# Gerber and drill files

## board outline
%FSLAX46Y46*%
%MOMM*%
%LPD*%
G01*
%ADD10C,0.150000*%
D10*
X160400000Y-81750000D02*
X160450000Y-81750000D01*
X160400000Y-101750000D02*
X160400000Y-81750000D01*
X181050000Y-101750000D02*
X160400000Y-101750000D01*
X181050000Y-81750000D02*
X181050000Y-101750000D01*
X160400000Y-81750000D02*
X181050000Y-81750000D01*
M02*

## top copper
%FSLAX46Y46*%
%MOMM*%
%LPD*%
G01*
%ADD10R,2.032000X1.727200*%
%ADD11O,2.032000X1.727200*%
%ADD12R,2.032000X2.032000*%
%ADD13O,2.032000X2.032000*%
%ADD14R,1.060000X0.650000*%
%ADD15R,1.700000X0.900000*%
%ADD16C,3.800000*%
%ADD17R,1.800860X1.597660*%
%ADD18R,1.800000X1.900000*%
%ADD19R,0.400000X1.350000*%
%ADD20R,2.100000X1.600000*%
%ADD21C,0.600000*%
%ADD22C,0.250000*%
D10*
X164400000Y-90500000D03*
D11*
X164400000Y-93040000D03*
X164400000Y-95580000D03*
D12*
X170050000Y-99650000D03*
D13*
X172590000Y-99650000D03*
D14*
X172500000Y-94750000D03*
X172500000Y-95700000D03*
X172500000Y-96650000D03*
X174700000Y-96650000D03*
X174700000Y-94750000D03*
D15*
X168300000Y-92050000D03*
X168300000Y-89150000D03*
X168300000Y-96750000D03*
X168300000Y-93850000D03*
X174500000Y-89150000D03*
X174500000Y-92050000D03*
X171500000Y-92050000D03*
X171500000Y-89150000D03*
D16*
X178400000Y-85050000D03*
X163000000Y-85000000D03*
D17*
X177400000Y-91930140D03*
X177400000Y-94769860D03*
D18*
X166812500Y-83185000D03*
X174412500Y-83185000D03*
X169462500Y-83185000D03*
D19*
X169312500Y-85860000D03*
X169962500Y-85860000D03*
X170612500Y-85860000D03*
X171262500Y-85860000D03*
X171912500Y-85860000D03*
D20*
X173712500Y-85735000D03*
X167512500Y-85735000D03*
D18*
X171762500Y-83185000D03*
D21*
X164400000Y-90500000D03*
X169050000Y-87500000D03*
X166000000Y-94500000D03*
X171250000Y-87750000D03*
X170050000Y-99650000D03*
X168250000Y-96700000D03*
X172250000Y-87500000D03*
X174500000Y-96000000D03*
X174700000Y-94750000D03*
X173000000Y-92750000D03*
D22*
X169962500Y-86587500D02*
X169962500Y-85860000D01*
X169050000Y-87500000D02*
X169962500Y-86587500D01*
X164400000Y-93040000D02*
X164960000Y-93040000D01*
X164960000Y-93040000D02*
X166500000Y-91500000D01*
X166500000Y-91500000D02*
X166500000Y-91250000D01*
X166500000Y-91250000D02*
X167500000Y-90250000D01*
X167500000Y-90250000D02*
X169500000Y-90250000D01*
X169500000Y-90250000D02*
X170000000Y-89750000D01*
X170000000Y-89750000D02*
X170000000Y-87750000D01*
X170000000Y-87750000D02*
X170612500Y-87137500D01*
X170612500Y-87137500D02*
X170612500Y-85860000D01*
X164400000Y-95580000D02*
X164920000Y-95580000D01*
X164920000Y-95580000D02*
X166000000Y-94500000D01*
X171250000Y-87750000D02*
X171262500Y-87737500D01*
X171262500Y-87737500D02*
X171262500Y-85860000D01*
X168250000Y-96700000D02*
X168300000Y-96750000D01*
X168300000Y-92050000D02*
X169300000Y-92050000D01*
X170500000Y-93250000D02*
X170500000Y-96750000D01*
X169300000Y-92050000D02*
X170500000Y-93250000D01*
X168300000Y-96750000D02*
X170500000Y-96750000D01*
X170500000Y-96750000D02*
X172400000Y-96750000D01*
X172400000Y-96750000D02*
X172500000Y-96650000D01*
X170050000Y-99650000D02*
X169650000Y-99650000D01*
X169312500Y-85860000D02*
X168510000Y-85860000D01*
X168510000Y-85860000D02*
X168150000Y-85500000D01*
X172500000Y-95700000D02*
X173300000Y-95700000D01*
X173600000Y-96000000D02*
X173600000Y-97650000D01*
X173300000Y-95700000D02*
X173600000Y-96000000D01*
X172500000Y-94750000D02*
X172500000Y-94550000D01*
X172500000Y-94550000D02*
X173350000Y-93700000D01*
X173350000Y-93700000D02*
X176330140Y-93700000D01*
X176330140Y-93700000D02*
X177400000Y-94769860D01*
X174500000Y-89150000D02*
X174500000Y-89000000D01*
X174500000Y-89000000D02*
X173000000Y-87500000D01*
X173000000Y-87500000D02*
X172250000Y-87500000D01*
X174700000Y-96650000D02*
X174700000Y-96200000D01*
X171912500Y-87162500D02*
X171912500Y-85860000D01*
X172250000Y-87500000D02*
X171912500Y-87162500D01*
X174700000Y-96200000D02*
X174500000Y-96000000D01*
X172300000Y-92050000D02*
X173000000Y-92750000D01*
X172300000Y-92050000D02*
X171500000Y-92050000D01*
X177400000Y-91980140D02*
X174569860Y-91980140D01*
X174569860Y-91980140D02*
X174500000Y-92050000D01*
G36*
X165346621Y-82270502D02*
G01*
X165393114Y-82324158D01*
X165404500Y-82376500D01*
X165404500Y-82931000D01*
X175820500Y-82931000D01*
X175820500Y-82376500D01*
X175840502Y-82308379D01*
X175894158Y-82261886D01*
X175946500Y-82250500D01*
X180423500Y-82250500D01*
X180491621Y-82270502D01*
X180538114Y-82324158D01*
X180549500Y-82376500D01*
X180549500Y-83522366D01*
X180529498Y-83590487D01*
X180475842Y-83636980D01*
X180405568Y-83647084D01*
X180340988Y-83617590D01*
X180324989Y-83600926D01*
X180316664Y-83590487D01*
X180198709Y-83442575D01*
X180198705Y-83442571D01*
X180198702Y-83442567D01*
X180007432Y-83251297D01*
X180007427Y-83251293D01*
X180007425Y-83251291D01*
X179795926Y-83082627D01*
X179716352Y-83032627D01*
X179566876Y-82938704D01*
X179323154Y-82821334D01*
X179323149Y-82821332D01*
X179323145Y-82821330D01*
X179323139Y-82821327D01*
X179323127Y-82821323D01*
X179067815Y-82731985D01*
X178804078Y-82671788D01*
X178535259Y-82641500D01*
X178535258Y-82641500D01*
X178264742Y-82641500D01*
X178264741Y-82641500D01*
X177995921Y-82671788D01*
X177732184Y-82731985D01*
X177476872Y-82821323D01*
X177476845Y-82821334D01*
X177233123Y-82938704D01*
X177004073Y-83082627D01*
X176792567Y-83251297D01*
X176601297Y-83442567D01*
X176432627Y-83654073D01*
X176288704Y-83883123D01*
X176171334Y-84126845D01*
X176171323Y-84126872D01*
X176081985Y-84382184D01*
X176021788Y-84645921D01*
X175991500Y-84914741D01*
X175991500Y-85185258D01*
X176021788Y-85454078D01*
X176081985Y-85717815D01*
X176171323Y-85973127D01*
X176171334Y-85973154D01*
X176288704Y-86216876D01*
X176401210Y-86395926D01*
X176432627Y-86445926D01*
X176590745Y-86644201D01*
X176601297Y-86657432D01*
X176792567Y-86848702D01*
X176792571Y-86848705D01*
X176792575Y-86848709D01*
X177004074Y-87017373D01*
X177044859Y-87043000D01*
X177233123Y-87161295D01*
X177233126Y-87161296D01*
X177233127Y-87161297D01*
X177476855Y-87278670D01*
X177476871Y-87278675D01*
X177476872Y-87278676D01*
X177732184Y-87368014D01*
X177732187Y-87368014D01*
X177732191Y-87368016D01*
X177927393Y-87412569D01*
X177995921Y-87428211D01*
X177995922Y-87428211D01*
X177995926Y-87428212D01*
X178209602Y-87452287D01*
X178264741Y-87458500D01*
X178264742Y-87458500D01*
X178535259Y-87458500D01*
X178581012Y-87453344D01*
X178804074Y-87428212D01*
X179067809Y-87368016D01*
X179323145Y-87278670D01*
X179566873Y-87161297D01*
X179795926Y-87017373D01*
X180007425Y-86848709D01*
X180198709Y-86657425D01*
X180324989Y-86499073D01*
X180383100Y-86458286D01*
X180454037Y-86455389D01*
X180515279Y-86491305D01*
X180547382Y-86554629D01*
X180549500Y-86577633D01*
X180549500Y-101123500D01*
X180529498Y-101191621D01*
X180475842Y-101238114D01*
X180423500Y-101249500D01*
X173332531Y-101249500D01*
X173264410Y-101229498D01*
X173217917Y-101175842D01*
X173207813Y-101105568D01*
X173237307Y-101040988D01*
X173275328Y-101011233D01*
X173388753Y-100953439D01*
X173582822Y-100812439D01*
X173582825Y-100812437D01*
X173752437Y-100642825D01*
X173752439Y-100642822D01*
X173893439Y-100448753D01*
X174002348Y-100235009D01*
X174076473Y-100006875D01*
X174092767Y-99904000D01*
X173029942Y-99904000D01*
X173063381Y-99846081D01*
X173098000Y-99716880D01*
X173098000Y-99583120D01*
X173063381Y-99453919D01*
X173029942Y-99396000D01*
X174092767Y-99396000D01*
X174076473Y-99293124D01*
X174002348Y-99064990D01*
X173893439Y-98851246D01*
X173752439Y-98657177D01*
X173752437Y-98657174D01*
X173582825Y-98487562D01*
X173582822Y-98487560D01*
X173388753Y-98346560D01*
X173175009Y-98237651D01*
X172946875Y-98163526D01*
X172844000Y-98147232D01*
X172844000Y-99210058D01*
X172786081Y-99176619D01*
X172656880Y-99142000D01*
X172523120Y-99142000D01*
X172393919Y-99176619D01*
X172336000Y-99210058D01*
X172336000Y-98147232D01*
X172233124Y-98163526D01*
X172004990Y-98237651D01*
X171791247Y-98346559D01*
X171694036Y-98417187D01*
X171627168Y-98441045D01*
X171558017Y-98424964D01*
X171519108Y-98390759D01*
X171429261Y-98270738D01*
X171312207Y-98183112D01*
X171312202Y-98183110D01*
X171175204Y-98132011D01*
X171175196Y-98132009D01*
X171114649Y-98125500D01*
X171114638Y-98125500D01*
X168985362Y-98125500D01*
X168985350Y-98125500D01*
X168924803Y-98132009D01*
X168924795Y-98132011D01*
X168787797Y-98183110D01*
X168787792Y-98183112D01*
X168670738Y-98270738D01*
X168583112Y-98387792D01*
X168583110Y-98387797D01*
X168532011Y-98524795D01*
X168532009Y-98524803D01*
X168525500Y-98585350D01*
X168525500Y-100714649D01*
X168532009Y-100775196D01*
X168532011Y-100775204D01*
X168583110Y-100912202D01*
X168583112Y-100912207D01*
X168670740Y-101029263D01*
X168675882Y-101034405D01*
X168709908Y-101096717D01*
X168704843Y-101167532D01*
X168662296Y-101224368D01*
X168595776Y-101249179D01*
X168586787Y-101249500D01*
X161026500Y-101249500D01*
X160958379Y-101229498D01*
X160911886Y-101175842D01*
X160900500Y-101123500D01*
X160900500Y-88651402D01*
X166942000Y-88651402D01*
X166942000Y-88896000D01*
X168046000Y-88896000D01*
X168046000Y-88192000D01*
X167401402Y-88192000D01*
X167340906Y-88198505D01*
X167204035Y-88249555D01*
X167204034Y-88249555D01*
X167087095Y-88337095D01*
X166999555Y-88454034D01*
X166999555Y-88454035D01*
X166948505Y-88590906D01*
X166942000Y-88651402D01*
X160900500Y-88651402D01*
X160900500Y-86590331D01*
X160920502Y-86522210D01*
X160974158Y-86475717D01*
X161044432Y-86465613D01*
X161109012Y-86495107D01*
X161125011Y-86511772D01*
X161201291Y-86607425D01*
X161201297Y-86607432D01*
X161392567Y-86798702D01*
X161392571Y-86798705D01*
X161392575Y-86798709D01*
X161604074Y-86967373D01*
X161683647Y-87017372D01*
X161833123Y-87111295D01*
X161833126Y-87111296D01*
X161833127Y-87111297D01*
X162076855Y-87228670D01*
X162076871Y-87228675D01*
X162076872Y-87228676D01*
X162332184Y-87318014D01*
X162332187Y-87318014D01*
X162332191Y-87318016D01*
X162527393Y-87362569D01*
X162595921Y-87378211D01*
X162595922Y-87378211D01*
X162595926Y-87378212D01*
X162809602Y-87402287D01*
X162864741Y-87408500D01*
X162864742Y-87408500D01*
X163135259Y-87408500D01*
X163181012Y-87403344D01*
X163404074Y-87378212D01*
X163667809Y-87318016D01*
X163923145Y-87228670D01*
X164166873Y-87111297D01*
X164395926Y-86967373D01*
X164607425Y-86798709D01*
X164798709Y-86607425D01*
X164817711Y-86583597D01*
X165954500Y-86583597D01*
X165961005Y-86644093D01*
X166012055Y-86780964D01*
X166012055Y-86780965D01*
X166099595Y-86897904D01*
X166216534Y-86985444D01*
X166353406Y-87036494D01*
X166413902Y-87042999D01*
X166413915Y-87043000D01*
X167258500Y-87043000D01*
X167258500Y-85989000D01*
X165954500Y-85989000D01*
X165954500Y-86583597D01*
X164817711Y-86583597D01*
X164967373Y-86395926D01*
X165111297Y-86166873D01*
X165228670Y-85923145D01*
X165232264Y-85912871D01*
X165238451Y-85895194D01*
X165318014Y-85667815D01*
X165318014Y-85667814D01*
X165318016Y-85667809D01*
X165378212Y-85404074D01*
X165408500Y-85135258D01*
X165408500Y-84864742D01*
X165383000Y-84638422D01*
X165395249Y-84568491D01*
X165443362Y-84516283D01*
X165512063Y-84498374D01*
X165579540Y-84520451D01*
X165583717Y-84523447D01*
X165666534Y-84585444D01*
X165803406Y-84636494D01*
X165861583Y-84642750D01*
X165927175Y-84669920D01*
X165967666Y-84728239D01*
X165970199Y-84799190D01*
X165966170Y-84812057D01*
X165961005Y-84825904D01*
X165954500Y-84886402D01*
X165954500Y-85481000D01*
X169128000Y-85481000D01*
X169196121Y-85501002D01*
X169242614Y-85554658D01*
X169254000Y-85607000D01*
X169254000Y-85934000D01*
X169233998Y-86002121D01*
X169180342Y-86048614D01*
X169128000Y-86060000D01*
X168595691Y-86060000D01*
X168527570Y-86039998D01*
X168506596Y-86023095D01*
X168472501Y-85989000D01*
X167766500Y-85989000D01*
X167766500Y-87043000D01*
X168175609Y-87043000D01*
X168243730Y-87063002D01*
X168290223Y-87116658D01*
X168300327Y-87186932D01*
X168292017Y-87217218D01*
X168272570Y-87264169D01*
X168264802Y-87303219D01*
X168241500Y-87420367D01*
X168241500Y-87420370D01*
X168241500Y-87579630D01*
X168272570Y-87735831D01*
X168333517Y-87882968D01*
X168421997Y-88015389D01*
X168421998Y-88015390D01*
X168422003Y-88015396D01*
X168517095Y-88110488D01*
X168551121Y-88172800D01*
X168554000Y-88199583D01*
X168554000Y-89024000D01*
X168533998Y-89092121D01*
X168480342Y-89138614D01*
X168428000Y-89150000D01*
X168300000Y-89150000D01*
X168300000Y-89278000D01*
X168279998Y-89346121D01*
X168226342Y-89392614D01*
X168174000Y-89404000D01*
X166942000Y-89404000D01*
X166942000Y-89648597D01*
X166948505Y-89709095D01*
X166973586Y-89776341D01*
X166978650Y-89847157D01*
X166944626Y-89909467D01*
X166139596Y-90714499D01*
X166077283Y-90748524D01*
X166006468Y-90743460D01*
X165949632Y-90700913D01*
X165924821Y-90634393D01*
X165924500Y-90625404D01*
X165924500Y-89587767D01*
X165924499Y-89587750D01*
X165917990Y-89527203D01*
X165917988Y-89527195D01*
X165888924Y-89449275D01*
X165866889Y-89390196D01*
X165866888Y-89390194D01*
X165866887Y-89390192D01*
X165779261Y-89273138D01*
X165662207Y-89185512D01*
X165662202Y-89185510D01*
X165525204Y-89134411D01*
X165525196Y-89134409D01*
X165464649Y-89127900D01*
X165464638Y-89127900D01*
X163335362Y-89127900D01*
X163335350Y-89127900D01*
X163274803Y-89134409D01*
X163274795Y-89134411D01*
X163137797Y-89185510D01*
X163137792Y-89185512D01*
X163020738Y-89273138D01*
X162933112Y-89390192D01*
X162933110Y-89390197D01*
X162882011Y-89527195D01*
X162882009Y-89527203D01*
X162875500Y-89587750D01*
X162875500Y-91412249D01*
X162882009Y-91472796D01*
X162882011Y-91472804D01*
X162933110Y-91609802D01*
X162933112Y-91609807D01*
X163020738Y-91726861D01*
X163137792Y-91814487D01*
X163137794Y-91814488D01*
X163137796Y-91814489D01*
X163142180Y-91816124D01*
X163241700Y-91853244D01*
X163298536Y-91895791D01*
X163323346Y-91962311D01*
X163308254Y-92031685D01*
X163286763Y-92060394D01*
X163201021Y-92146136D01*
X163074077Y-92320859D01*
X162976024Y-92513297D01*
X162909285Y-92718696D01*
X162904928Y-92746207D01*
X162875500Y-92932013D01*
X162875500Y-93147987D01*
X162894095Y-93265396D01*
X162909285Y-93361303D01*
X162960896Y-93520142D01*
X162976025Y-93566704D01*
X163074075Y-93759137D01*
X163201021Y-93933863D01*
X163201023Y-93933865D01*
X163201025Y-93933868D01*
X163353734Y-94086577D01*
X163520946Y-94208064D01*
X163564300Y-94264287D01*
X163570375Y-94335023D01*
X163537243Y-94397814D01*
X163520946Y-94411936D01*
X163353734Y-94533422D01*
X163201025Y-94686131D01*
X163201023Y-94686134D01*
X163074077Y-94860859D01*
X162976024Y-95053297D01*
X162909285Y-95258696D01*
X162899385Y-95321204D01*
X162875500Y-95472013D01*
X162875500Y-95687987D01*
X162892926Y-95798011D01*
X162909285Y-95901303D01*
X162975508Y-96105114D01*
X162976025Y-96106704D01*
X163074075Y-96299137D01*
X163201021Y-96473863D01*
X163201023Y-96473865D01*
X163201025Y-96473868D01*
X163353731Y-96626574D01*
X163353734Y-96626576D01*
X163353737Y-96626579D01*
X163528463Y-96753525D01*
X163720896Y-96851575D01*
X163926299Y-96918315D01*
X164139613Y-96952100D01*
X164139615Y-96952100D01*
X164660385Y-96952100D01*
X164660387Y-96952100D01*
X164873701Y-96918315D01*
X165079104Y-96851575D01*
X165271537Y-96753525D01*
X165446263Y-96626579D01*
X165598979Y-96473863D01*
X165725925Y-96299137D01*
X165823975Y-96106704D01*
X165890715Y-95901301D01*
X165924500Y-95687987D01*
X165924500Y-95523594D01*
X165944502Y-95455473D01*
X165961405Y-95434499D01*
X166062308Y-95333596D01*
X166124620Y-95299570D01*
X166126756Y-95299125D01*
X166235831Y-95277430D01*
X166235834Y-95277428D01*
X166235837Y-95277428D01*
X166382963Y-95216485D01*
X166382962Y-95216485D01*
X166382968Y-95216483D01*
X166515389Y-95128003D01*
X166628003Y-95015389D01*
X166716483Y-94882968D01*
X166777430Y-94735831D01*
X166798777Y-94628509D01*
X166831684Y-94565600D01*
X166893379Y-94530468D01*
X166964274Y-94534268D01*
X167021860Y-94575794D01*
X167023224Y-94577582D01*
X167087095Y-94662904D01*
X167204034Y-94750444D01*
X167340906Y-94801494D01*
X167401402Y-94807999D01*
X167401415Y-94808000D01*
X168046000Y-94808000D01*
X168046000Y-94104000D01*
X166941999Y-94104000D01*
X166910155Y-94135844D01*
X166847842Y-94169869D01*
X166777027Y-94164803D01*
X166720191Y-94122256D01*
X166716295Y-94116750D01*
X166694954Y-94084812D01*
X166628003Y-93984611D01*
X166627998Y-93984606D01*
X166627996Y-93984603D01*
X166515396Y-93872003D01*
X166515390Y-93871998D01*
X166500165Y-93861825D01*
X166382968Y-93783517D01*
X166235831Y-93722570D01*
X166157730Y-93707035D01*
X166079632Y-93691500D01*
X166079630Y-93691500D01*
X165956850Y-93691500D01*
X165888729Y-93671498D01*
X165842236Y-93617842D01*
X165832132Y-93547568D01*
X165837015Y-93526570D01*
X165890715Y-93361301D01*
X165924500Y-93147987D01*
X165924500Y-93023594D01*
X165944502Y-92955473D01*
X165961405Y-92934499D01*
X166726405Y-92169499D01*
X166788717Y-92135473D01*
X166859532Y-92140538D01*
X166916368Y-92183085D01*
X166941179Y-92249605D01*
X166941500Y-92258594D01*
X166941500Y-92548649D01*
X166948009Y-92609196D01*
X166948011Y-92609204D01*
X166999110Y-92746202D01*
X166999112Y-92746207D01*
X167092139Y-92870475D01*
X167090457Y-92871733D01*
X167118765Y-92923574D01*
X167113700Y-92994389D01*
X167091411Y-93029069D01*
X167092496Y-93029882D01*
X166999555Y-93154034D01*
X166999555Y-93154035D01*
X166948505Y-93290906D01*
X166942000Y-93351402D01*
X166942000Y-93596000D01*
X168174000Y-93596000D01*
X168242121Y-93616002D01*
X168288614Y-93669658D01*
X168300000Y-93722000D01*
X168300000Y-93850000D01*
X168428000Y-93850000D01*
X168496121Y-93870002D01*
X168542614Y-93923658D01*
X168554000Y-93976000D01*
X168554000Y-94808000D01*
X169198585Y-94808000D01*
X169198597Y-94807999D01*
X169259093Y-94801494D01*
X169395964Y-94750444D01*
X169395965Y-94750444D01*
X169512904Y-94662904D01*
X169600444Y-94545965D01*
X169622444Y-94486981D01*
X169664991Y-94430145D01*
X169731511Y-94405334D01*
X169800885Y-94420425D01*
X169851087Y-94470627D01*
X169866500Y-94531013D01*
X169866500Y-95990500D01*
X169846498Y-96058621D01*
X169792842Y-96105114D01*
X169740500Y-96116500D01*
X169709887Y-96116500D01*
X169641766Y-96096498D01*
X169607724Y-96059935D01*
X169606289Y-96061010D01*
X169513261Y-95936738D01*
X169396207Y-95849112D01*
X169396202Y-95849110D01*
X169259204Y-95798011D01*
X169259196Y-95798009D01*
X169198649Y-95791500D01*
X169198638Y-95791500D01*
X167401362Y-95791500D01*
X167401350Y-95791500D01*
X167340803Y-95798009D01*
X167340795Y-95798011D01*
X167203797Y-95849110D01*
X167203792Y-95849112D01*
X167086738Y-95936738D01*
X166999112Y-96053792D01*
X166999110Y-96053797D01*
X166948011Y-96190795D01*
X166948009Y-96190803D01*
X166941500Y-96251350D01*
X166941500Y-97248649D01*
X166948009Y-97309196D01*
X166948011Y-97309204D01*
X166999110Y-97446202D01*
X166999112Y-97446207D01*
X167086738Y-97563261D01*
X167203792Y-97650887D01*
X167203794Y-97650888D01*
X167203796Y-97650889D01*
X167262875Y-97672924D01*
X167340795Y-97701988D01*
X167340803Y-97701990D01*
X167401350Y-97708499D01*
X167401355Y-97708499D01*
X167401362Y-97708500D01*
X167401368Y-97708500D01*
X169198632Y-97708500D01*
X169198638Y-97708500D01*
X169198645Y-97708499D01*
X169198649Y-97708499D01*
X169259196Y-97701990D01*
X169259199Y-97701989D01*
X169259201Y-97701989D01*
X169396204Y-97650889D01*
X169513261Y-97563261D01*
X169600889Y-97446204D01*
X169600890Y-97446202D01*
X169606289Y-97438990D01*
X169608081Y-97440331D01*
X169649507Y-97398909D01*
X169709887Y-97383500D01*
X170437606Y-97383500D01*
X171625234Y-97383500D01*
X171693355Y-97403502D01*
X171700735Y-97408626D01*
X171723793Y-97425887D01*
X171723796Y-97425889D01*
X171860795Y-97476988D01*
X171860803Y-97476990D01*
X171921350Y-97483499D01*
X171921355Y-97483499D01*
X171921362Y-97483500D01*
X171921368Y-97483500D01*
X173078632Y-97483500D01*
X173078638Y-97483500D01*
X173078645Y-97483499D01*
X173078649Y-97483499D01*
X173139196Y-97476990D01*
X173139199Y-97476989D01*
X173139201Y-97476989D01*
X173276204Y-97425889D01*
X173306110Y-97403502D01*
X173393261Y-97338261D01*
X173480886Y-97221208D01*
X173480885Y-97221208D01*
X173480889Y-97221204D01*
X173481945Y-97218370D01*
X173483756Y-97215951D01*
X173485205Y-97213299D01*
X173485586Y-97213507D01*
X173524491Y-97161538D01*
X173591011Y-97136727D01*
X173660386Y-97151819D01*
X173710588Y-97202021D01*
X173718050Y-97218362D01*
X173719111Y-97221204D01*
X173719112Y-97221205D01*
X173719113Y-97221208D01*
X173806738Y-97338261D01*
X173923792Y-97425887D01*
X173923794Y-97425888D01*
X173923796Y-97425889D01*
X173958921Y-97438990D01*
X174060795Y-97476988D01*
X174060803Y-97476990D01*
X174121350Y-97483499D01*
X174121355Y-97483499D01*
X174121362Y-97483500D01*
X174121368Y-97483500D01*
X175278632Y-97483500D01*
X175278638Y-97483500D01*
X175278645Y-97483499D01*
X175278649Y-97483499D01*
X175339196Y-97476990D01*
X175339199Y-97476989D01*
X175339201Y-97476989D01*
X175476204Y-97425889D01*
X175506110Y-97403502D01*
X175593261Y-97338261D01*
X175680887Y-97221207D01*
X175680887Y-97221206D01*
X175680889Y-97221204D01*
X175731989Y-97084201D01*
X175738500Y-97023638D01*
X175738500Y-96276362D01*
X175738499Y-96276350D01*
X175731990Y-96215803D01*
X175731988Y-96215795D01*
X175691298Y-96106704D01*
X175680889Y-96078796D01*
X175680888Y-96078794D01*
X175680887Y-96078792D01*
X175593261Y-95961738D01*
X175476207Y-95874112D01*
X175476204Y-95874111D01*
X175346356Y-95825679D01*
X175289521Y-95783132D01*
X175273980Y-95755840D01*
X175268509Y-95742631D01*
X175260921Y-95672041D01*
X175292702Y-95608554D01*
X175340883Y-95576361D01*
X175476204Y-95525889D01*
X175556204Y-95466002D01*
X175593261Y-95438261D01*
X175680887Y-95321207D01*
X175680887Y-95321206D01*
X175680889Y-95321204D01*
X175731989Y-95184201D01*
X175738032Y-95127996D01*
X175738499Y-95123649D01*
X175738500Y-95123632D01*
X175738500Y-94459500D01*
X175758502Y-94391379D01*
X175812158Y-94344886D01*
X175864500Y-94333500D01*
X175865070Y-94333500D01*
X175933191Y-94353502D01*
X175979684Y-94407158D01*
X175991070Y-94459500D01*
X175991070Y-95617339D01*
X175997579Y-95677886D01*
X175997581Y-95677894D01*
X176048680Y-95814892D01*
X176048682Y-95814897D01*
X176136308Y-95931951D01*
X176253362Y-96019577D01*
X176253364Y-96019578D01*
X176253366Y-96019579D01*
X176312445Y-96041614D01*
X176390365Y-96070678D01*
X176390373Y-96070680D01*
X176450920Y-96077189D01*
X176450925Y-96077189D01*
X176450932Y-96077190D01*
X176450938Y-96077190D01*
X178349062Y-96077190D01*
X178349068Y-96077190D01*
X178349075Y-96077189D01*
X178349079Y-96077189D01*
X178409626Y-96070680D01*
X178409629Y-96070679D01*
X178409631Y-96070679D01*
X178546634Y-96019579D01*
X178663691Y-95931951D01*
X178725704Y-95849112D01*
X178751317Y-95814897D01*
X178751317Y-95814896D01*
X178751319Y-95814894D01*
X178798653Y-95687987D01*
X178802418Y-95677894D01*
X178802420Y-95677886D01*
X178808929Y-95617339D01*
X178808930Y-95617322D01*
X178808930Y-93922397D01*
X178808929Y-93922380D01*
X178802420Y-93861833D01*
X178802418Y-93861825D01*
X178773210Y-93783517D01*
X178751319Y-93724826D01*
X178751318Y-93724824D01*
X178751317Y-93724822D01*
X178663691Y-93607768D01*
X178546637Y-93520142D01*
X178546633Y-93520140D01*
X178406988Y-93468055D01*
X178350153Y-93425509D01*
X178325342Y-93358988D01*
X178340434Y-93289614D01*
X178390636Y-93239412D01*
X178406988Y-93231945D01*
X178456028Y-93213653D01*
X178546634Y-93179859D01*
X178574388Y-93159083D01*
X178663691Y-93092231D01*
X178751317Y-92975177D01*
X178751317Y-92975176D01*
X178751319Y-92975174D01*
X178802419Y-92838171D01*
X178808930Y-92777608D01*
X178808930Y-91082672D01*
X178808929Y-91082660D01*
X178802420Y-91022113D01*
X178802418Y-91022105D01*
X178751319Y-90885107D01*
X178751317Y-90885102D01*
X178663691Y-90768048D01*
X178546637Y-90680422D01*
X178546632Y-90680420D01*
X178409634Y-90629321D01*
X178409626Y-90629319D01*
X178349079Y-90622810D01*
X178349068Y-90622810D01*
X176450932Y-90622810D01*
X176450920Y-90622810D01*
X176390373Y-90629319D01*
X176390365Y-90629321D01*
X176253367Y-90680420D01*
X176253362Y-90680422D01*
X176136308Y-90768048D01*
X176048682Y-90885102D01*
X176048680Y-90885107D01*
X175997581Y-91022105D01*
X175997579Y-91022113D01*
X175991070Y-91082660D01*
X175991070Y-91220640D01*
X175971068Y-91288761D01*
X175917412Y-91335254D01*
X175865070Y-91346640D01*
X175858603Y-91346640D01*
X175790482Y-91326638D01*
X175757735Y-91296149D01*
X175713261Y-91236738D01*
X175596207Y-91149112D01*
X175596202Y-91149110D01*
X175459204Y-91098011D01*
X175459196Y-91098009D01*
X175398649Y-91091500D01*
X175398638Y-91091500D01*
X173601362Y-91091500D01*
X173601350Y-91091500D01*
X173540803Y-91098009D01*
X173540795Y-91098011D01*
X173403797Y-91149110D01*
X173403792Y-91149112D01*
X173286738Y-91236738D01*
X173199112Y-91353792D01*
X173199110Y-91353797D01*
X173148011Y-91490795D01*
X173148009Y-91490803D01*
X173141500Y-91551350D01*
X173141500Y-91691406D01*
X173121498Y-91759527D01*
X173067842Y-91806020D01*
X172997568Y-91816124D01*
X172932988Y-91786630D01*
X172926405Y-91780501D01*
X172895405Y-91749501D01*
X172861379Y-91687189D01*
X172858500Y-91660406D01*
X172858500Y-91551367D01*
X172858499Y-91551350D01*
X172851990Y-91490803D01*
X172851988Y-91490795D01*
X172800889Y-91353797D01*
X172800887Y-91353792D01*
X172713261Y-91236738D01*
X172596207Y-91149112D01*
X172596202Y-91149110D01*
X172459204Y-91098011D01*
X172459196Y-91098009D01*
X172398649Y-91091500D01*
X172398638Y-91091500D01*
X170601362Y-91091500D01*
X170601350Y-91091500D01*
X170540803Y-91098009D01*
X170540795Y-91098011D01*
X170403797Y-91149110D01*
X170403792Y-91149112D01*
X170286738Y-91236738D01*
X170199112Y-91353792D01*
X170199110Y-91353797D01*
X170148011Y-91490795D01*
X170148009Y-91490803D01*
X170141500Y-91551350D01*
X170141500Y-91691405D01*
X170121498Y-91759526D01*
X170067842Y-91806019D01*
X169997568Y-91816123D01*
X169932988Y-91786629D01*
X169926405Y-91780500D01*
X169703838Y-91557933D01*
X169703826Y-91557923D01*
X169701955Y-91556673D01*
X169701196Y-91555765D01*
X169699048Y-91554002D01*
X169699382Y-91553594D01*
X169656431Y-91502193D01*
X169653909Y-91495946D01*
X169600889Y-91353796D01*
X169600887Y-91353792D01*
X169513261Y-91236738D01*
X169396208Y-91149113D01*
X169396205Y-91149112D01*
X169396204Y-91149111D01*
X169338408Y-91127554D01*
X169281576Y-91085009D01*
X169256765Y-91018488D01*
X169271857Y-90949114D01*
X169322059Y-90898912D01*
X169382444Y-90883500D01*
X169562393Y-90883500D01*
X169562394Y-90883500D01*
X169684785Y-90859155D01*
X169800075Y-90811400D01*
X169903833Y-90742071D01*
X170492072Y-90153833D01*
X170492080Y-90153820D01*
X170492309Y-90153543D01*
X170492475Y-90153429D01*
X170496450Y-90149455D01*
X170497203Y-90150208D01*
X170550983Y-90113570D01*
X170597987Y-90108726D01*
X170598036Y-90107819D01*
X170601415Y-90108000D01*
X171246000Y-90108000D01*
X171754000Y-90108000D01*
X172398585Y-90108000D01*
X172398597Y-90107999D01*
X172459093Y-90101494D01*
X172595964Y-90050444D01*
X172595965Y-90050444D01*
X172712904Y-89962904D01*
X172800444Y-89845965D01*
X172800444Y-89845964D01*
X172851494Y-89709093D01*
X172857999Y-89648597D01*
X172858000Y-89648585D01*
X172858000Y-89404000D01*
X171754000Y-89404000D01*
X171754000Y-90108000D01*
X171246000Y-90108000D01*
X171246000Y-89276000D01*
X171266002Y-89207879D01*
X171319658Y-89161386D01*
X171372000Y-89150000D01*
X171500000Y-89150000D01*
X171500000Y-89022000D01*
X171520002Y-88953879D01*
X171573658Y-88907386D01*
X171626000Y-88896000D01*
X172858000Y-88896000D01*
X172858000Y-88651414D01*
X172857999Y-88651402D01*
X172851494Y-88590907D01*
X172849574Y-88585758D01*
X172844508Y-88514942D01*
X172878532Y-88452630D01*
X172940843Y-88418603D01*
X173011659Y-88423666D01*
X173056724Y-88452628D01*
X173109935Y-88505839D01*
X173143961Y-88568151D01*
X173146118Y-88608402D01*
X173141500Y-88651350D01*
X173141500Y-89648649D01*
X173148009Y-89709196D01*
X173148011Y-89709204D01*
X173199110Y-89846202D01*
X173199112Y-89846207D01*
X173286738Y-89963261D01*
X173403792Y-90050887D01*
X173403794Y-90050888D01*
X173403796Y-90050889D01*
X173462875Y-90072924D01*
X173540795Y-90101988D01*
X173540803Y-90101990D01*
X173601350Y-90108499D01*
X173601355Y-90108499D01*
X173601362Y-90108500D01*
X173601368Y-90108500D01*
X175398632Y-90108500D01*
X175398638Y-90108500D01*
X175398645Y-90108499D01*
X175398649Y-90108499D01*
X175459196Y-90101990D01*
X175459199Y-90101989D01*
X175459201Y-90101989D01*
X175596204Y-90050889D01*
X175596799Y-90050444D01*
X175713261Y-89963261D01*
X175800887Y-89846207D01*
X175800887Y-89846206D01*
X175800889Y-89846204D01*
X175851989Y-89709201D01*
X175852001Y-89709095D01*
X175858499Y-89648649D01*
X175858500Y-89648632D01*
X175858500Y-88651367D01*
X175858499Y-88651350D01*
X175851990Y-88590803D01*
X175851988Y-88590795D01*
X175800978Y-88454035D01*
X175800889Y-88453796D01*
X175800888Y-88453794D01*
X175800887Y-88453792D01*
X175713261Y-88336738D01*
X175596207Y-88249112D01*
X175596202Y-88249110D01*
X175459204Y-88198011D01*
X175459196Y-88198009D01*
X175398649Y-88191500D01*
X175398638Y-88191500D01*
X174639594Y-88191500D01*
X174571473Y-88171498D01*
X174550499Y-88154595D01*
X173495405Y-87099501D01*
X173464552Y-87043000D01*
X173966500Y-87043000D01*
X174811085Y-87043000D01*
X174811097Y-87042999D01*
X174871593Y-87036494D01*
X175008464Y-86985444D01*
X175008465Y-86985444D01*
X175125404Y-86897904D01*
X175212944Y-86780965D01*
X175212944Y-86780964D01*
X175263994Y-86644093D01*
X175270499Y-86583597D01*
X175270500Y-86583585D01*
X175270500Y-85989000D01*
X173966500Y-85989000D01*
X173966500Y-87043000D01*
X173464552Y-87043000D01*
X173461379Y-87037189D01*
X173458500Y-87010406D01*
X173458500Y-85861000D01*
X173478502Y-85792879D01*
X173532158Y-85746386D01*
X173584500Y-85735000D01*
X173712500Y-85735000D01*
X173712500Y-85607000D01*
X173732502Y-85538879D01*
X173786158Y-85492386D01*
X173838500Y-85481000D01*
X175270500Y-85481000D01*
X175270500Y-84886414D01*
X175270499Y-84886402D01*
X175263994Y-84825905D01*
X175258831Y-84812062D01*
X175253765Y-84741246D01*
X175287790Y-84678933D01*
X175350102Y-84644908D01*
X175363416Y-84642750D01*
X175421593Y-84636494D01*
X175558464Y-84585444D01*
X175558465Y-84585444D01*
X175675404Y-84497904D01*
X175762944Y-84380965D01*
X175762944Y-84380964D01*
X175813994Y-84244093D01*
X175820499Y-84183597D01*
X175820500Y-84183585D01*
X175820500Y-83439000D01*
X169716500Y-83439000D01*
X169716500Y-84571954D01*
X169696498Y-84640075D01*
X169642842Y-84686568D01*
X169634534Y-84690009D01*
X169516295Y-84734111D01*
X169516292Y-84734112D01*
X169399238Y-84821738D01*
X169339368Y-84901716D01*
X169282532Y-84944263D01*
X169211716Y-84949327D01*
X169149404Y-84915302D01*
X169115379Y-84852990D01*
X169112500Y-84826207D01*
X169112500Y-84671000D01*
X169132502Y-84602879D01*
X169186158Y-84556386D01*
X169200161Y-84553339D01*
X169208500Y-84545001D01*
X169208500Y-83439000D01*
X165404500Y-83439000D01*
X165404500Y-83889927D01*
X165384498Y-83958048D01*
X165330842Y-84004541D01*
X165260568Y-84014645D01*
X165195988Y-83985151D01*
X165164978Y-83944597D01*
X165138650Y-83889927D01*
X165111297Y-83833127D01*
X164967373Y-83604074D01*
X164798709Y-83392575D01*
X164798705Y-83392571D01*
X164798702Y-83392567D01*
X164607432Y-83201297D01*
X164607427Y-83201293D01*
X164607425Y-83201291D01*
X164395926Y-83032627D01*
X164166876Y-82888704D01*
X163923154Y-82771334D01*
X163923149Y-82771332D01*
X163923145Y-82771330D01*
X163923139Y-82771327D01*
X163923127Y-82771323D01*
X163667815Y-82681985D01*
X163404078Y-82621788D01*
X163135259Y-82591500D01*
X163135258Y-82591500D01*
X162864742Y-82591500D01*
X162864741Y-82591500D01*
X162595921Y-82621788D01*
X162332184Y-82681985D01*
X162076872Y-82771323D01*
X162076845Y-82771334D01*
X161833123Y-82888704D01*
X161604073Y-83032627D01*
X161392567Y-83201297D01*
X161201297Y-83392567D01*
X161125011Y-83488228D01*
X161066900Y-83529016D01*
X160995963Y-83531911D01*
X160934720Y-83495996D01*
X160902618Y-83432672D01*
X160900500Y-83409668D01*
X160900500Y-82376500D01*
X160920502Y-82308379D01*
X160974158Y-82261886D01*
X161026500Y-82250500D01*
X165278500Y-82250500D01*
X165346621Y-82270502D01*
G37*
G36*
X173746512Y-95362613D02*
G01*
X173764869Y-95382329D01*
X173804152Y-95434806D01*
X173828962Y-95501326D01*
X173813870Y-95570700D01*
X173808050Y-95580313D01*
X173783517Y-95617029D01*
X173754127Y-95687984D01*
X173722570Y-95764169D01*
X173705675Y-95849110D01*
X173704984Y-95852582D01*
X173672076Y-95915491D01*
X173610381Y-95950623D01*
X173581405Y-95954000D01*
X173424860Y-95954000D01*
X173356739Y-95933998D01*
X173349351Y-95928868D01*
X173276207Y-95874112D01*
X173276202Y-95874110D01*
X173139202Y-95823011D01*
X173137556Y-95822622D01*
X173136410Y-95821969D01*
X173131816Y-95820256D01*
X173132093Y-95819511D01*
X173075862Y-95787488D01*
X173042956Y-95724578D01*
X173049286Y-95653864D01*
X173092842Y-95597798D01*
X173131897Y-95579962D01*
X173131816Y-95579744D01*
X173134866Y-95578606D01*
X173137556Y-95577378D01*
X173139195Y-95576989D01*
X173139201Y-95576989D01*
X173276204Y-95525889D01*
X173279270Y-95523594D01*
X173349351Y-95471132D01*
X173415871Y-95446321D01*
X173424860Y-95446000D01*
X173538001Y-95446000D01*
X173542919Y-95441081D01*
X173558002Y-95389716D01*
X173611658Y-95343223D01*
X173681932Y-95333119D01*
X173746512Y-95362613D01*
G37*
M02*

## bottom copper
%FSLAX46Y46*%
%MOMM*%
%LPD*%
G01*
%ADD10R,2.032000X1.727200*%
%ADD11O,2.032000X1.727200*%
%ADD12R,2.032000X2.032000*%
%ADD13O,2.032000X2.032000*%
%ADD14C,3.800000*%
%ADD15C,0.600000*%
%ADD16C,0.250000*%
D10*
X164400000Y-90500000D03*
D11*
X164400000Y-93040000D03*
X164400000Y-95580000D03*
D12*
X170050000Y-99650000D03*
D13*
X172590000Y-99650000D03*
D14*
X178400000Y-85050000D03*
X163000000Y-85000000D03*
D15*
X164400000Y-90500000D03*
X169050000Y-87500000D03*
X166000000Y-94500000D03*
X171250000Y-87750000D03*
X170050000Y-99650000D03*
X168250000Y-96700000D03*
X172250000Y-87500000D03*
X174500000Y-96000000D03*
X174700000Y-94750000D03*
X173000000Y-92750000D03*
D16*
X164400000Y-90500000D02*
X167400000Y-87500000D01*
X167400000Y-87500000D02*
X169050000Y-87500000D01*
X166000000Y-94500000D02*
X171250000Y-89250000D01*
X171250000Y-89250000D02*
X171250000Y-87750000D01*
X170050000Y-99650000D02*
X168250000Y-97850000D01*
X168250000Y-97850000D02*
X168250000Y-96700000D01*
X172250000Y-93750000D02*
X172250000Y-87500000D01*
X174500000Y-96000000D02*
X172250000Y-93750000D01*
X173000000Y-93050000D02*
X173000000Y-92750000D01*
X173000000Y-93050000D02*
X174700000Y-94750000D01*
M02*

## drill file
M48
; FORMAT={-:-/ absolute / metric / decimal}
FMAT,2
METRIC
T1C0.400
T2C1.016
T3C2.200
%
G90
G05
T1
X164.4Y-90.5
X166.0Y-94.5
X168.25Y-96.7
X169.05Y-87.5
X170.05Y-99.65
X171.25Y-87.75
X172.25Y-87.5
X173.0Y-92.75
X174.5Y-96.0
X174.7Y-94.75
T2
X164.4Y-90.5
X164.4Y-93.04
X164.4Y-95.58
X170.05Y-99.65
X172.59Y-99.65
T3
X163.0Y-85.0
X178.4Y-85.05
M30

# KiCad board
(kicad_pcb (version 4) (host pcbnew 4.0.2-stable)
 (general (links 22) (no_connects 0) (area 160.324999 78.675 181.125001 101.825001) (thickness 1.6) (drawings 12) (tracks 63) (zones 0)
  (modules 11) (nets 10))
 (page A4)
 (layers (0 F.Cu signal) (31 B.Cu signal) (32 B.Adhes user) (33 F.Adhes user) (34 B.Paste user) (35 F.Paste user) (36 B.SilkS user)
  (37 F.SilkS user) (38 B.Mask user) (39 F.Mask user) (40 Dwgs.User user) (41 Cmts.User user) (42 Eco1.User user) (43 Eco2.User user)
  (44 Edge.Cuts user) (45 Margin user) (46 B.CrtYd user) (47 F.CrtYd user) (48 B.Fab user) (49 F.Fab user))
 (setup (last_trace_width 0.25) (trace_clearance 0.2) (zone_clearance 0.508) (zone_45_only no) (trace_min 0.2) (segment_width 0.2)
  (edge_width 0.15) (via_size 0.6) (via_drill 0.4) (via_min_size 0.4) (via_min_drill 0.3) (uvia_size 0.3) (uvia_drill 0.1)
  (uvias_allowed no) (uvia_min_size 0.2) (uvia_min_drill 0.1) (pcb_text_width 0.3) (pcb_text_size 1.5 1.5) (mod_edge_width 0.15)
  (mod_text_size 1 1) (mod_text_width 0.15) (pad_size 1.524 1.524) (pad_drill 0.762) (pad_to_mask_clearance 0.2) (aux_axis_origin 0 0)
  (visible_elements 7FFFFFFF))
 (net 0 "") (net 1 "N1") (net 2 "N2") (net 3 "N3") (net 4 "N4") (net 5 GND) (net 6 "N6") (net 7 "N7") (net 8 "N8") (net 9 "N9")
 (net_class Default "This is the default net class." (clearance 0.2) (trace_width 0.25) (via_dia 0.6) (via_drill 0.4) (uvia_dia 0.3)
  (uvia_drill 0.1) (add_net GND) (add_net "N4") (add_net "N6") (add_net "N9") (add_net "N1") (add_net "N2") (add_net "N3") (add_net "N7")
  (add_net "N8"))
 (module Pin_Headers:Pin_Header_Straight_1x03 (layer F.Cu) (at 164.4 90.5)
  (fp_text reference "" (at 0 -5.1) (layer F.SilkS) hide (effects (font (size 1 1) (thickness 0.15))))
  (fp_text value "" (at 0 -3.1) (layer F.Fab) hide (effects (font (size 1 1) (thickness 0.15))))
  (pad 1 thru_hole rect (at 0 0) (size 2.032 1.7272) (drill 1.016) (layers *.Cu *.Mask F.SilkS) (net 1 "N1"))
  (pad 2 thru_hole oval (at 0 2.54) (size 2.032 1.7272) (drill 1.016) (layers *.Cu *.Mask F.SilkS) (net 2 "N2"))
  (pad 3 thru_hole oval (at 0 5.08) (size 2.032 1.7272) (drill 1.016) (layers *.Cu *.Mask F.SilkS) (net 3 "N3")))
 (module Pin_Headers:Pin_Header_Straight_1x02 (layer F.Cu) (at 170.05 99.65 90)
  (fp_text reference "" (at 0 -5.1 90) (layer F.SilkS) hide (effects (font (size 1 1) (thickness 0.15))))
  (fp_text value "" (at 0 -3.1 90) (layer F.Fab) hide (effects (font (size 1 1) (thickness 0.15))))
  (pad 1 thru_hole rect (at 0 0 90) (size 2.032 2.032) (drill 1.016) (layers *.Cu *.Mask F.SilkS) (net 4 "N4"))
  (pad 2 thru_hole oval (at 0 2.54 90) (size 2.032 2.032) (drill 1.016) (layers *.Cu *.Mask F.SilkS) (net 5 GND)))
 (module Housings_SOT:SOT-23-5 (layer F.Cu) (at 173.6 95.7) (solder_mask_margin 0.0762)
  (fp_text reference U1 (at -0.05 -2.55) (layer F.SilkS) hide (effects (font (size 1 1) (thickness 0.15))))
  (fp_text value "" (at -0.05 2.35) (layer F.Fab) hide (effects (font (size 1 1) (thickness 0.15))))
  (pad 1 smd rect (at -1.1 -0.95) (size 1.06 0.65) (layers F.Cu F.Paste F.Mask) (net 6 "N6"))
  (pad 2 smd rect (at -1.1 0) (size 1.06 0.65) (layers F.Cu F.Paste F.Mask) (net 5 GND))
  (pad 3 smd rect (at -1.1 0.95) (size 1.06 0.65) (layers F.Cu F.Paste F.Mask) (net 4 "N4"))
  (pad 4 smd rect (at 1.1 0.95) (size 1.06 0.65) (layers F.Cu F.Paste F.Mask) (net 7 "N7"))
  (pad 5 smd rect (at 1.1 -0.95) (size 1.06 0.65) (layers F.Cu F.Paste F.Mask) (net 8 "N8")))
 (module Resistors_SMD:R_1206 (layer F.Cu) (at 168.3 90.6 90)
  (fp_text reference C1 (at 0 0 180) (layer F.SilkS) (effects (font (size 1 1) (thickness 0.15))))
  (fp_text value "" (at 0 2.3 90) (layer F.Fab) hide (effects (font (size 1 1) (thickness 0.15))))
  (pad 1 smd rect (at -1.45 0 90) (size 0.9 1.7) (layers F.Cu F.Paste F.Mask) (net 4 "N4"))
  (pad 2 smd rect (at 1.45 0 90) (size 0.9 1.7) (layers F.Cu F.Paste F.Mask) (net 5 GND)))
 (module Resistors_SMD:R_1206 (layer F.Cu) (at 168.3 95.3 90)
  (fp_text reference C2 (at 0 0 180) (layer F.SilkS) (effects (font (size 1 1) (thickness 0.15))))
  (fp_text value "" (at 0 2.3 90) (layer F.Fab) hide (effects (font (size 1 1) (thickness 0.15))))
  (pad 1 smd rect (at -1.45 0 90) (size 0.9 1.7) (layers F.Cu F.Paste F.Mask) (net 4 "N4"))
  (pad 2 smd rect (at 1.45 0 90) (size 0.9 1.7) (layers F.Cu F.Paste F.Mask) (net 5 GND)))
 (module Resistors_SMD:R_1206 (layer F.Cu) (at 174.5 90.6 270)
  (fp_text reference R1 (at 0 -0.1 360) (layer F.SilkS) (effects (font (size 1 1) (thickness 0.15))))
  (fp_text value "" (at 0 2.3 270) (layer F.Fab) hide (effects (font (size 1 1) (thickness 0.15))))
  (pad 1 smd rect (at -1.45 0 270) (size 0.9 1.7) (layers F.Cu F.Paste F.Mask) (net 7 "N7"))
  (pad 2 smd rect (at 1.45 0 270) (size 0.9 1.7) (layers F.Cu F.Paste F.Mask) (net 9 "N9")))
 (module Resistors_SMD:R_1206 (layer F.Cu) (at 171.5 90.6 90)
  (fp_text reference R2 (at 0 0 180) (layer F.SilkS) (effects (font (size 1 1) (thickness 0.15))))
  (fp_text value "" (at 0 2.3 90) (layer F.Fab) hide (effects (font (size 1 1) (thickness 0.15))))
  (pad 1 smd rect (at -1.45 0 90) (size 0.9 1.7) (layers F.Cu F.Paste F.Mask) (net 8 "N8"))
  (pad 2 smd rect (at 1.45 0 90) (size 0.9 1.7) (layers F.Cu F.Paste F.Mask) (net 5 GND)))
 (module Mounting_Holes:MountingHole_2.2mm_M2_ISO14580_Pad (layer F.Cu) (at 178.4 85.05)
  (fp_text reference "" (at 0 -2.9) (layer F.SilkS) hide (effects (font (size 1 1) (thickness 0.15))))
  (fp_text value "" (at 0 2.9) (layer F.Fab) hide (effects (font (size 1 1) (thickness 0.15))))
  (pad 1 thru_hole circle (at 0 0) (size 3.8 3.8) (drill 2.2) (layers *.Cu *.Mask F.SilkS)))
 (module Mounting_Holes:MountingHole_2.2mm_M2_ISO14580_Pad (layer F.Cu) (at 163 85)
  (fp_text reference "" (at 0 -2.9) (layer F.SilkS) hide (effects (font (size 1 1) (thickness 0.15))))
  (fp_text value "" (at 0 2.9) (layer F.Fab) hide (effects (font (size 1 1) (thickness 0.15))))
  (pad 1 thru_hole circle (at 0 0) (size 3.8 3.8) (drill 2.2) (layers *.Cu *.Mask F.SilkS)))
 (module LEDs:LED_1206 (layer F.Cu) (at 177.4 93.35 90)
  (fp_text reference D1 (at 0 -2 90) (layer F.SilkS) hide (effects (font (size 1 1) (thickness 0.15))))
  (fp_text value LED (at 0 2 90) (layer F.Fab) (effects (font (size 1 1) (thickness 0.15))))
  (pad 2 smd rect (at 1.41986 0 270) (size 1.59766 1.80086) (layers F.Cu F.Paste F.Mask) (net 9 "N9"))
  (pad 1 smd rect (at -1.41986 0 270) (size 1.59766 1.80086) (layers F.Cu F.Paste F.Mask) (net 6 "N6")))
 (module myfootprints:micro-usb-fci (layer F.Cu) (at 171.2 84.2) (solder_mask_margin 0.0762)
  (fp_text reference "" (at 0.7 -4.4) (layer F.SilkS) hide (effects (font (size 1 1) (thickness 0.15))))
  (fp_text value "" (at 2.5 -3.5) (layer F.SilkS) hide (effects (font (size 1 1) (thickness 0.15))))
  (pad 6 smd rect (at -4.3875 -1.015) (size 1.8 1.9) (layers F.Cu F.Paste F.Mask) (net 5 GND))
  (pad 6 smd rect (at 3.2125 -1.015) (size 1.8 1.9) (layers F.Cu F.Paste F.Mask) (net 5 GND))
  (pad 6 smd rect (at -1.7375 -1.015) (size 1.8 1.9) (layers F.Cu F.Paste F.Mask) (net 5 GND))
  (pad 5 smd rect (at -1.8875 1.66) (size 0.4 1.35) (layers F.Cu F.Paste F.Mask) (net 5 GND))
  (pad 4 smd rect (at -1.2375 1.66) (size 0.4 1.35) (layers F.Cu F.Paste F.Mask) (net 1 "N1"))
  (pad 3 smd rect (at -0.5875 1.66) (size 0.4 1.35) (layers F.Cu F.Paste F.Mask) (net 2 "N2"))
  (pad 2 smd rect (at 0.0625 1.66) (size 0.4 1.35) (layers F.Cu F.Paste F.Mask) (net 3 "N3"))
  (pad 1 smd rect (at 0.7125 1.66) (size 0.4 1.35) (layers F.Cu F.Paste F.Mask) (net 7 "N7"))
  (pad 6 smd rect (at 2.5125 1.535) (size 2.1 1.6) (layers F.Cu F.Paste F.Mask) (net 5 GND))
  (pad 6 smd rect (at -3.6875 1.535) (size 2.1 1.6) (layers F.Cu F.Paste F.Mask) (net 5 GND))
  (pad 6 smd rect (at 0.5625 -1.015) (size 1.8 1.9) (layers F.Cu F.Paste F.Mask) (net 5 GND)))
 (gr_line (start 160.4 81.75) (end 160.45 81.75) (angle 90) (layer Edge.Cuts) (width 0.15))
 (gr_line (start 160.4 101.75) (end 160.4 81.75) (angle 90) (layer Edge.Cuts) (width 0.15))
 (gr_line (start 181.05 101.75) (end 160.4 101.75) (angle 90) (layer Edge.Cuts) (width 0.15))
 (gr_line (start 181.05 81.75) (end 181.05 101.75) (angle 90) (layer Edge.Cuts) (width 0.15))
 (gr_line (start 160.4 81.75) (end 181.05 81.75) (angle 90) (layer Edge.Cuts) (width 0.15))
 (via (at 164.4 90.5) (size 0.6) (drill 0.4) (layers F.Cu B.Cu) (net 1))
 (segment (start 164.4 90.5) (end 167.4 87.5) (width 0.25) (layer B.Cu) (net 1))
 (segment (start 169.9625 86.5875) (end 169.9625 85.86) (width 0.25) (layer F.Cu) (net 1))
 (segment (start 169.05 87.5) (end 169.9625 86.5875) (width 0.25) (layer F.Cu) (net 1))
 (via (at 169.05 87.5) (size 0.6) (drill 0.4) (layers F.Cu B.Cu) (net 1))
 (segment (start 167.4 87.5) (end 169.05 87.5) (width 0.25) (layer B.Cu) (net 1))
 (segment (start 164.4 93.04) (end 164.96 93.04) (width 0.25) (layer F.Cu) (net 2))
 (segment (start 164.96 93.04) (end 166.5 91.5) (width 0.25) (layer F.Cu) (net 2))
 (segment (start 166.5 91.5) (end 166.5 91.25) (width 0.25) (layer F.Cu) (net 2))
 (segment (start 166.5 91.25) (end 167.5 90.25) (width 0.25) (layer F.Cu) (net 2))
 (segment (start 167.5 90.25) (end 169.5 90.25) (width 0.25) (layer F.Cu) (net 2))
 (segment (start 169.5 90.25) (end 170 89.75) (width 0.25) (layer F.Cu) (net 2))
 (segment (start 170 89.75) (end 170 87.75) (width 0.25) (layer F.Cu) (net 2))
 (segment (start 170 87.75) (end 170.6125 87.1375) (width 0.25) (layer F.Cu) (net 2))
 (segment (start 170.6125 87.1375) (end 170.6125 85.86) (width 0.25) (layer F.Cu) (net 2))
 (segment (start 164.4 95.58) (end 164.92 95.58) (width 0.25) (layer F.Cu) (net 3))
 (segment (start 164.92 95.58) (end 166 94.5) (width 0.25) (layer F.Cu) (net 3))
 (via (at 166 94.5) (size 0.6) (drill 0.4) (layers F.Cu B.Cu) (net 3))
 (segment (start 166 94.5) (end 171.25 89.25) (width 0.25) (layer B.Cu) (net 3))
 (segment (start 171.25 89.25) (end 171.25 87.75) (width 0.25) (layer B.Cu) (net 3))
 (via (at 171.25 87.75) (size 0.6) (drill 0.4) (layers F.Cu B.Cu) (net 3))
 (segment (start 171.25 87.75) (end 171.2625 87.7375) (width 0.25) (layer F.Cu) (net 3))
 (segment (start 171.2625 87.7375) (end 171.2625 85.86) (width 0.25) (layer F.Cu) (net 3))
 (via (at 170.05 99.65) (size 0.6) (drill 0.4) (layers F.Cu B.Cu) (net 4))
 (segment (start 170.05 99.65) (end 168.25 97.85) (width 0.25) (layer B.Cu) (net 4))
 (segment (start 168.25 96.7) (end 168.3 96.75) (width 0.25) (layer F.Cu) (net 4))
 (via (at 168.25 96.7) (size 0.6) (drill 0.4) (layers F.Cu B.Cu) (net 4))
 (segment (start 168.25 97.85) (end 168.25 96.7) (width 0.25) (layer B.Cu) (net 4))
 (segment (start 168.3 92.05) (end 169.3 92.05) (width 0.25) (layer F.Cu) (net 4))
 (segment (start 170.5 93.25) (end 170.5 96.75) (width 0.25) (layer F.Cu) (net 4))
 (segment (start 169.3 92.05) (end 170.5 93.25) (width 0.25) (layer F.Cu) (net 4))
 (segment (start 168.3 96.75) (end 170.5 96.75) (width 0.25) (layer F.Cu) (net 4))
 (segment (start 170.5 96.75) (end 172.4 96.75) (width 0.25) (layer F.Cu) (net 4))
 (segment (start 172.4 96.75) (end 172.5 96.65) (width 0.25) (layer F.Cu) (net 4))
 (segment (start 170.05 99.65) (end 169.65 99.65) (width 0.25) (layer F.Cu) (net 4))
 (segment (start 169.3125 85.86) (end 168.51 85.86) (width 0.25) (layer F.Cu) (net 5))
 (segment (start 168.51 85.86) (end 168.15 85.5) (width 0.25) (layer F.Cu) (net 5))
 (segment (start 172.5 95.7) (end 173.3 95.7) (width 0.25) (layer F.Cu) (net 5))
 (segment (start 173.6 96) (end 173.6 97.65) (width 0.25) (layer F.Cu) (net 5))
 (segment (start 173.3 95.7) (end 173.6 96) (width 0.25) (layer F.Cu) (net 5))
 (segment (start 172.5 94.75) (end 172.5 94.55) (width 0.25) (layer F.Cu) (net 6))
 (segment (start 172.5 94.55) (end 173.35 93.7) (width 0.25) (layer F.Cu) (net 6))
 (segment (start 173.35 93.7) (end 176.33014 93.7) (width 0.25) (layer F.Cu) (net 6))
 (segment (start 176.33014 93.7) (end 177.4 94.76986) (width 0.25) (layer F.Cu) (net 6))
 (segment (start 174.5 89.15) (end 174.5 89) (width 0.25) (layer F.Cu) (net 7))
 (segment (start 174.5 89) (end 173 87.5) (width 0.25) (layer F.Cu) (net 7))
 (segment (start 173 87.5) (end 172.25 87.5) (width 0.25) (layer F.Cu) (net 7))
 (segment (start 174.7 96.65) (end 174.7 96.2) (width 0.25) (layer F.Cu) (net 7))
 (segment (start 171.9125 87.1625) (end 171.9125 85.86) (width 0.25) (layer F.Cu) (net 7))
 (segment (start 172.25 87.5) (end 171.9125 87.1625) (width 0.25) (layer F.Cu) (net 7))
 (via (at 172.25 87.5) (size 0.6) (drill 0.4) (layers F.Cu B.Cu) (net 7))
 (segment (start 172.25 93.75) (end 172.25 87.5) (width 0.25) (layer B.Cu) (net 7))
 (segment (start 174.5 96) (end 172.25 93.75) (width 0.25) (layer B.Cu) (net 7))
 (via (at 174.5 96) (size 0.6) (drill 0.4) (layers F.Cu B.Cu) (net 7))
 (segment (start 174.7 96.2) (end 174.5 96) (width 0.25) (layer F.Cu) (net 7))
 (via (at 174.7 94.75) (size 0.6) (drill 0.4) (layers F.Cu B.Cu) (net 8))
 (segment (start 172.3 92.05) (end 173 92.75) (width 0.25) (layer F.Cu) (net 8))
 (via (at 173 92.75) (size 0.6) (drill 0.4) (layers F.Cu B.Cu) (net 8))
 (segment (start 173 93.05) (end 173 92.75) (width 0.25) (layer B.Cu) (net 8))
 (segment (start 173 93.05) (end 174.7 94.75) (width 0.25) (layer B.Cu) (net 8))
 (segment (start 172.3 92.05) (end 171.5 92.05) (width 0.25) (layer F.Cu) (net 8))
 (segment (start 177.4 91.98014) (end 174.56986 91.98014) (width 0.25) (layer F.Cu) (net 9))
 (segment (start 174.56986 91.98014) (end 174.5 92.05) (width 0.25) (layer F.Cu) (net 9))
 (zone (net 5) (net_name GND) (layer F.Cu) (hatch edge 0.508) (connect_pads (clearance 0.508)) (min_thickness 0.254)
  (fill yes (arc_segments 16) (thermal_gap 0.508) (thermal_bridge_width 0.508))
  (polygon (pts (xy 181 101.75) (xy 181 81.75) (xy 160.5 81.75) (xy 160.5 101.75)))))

